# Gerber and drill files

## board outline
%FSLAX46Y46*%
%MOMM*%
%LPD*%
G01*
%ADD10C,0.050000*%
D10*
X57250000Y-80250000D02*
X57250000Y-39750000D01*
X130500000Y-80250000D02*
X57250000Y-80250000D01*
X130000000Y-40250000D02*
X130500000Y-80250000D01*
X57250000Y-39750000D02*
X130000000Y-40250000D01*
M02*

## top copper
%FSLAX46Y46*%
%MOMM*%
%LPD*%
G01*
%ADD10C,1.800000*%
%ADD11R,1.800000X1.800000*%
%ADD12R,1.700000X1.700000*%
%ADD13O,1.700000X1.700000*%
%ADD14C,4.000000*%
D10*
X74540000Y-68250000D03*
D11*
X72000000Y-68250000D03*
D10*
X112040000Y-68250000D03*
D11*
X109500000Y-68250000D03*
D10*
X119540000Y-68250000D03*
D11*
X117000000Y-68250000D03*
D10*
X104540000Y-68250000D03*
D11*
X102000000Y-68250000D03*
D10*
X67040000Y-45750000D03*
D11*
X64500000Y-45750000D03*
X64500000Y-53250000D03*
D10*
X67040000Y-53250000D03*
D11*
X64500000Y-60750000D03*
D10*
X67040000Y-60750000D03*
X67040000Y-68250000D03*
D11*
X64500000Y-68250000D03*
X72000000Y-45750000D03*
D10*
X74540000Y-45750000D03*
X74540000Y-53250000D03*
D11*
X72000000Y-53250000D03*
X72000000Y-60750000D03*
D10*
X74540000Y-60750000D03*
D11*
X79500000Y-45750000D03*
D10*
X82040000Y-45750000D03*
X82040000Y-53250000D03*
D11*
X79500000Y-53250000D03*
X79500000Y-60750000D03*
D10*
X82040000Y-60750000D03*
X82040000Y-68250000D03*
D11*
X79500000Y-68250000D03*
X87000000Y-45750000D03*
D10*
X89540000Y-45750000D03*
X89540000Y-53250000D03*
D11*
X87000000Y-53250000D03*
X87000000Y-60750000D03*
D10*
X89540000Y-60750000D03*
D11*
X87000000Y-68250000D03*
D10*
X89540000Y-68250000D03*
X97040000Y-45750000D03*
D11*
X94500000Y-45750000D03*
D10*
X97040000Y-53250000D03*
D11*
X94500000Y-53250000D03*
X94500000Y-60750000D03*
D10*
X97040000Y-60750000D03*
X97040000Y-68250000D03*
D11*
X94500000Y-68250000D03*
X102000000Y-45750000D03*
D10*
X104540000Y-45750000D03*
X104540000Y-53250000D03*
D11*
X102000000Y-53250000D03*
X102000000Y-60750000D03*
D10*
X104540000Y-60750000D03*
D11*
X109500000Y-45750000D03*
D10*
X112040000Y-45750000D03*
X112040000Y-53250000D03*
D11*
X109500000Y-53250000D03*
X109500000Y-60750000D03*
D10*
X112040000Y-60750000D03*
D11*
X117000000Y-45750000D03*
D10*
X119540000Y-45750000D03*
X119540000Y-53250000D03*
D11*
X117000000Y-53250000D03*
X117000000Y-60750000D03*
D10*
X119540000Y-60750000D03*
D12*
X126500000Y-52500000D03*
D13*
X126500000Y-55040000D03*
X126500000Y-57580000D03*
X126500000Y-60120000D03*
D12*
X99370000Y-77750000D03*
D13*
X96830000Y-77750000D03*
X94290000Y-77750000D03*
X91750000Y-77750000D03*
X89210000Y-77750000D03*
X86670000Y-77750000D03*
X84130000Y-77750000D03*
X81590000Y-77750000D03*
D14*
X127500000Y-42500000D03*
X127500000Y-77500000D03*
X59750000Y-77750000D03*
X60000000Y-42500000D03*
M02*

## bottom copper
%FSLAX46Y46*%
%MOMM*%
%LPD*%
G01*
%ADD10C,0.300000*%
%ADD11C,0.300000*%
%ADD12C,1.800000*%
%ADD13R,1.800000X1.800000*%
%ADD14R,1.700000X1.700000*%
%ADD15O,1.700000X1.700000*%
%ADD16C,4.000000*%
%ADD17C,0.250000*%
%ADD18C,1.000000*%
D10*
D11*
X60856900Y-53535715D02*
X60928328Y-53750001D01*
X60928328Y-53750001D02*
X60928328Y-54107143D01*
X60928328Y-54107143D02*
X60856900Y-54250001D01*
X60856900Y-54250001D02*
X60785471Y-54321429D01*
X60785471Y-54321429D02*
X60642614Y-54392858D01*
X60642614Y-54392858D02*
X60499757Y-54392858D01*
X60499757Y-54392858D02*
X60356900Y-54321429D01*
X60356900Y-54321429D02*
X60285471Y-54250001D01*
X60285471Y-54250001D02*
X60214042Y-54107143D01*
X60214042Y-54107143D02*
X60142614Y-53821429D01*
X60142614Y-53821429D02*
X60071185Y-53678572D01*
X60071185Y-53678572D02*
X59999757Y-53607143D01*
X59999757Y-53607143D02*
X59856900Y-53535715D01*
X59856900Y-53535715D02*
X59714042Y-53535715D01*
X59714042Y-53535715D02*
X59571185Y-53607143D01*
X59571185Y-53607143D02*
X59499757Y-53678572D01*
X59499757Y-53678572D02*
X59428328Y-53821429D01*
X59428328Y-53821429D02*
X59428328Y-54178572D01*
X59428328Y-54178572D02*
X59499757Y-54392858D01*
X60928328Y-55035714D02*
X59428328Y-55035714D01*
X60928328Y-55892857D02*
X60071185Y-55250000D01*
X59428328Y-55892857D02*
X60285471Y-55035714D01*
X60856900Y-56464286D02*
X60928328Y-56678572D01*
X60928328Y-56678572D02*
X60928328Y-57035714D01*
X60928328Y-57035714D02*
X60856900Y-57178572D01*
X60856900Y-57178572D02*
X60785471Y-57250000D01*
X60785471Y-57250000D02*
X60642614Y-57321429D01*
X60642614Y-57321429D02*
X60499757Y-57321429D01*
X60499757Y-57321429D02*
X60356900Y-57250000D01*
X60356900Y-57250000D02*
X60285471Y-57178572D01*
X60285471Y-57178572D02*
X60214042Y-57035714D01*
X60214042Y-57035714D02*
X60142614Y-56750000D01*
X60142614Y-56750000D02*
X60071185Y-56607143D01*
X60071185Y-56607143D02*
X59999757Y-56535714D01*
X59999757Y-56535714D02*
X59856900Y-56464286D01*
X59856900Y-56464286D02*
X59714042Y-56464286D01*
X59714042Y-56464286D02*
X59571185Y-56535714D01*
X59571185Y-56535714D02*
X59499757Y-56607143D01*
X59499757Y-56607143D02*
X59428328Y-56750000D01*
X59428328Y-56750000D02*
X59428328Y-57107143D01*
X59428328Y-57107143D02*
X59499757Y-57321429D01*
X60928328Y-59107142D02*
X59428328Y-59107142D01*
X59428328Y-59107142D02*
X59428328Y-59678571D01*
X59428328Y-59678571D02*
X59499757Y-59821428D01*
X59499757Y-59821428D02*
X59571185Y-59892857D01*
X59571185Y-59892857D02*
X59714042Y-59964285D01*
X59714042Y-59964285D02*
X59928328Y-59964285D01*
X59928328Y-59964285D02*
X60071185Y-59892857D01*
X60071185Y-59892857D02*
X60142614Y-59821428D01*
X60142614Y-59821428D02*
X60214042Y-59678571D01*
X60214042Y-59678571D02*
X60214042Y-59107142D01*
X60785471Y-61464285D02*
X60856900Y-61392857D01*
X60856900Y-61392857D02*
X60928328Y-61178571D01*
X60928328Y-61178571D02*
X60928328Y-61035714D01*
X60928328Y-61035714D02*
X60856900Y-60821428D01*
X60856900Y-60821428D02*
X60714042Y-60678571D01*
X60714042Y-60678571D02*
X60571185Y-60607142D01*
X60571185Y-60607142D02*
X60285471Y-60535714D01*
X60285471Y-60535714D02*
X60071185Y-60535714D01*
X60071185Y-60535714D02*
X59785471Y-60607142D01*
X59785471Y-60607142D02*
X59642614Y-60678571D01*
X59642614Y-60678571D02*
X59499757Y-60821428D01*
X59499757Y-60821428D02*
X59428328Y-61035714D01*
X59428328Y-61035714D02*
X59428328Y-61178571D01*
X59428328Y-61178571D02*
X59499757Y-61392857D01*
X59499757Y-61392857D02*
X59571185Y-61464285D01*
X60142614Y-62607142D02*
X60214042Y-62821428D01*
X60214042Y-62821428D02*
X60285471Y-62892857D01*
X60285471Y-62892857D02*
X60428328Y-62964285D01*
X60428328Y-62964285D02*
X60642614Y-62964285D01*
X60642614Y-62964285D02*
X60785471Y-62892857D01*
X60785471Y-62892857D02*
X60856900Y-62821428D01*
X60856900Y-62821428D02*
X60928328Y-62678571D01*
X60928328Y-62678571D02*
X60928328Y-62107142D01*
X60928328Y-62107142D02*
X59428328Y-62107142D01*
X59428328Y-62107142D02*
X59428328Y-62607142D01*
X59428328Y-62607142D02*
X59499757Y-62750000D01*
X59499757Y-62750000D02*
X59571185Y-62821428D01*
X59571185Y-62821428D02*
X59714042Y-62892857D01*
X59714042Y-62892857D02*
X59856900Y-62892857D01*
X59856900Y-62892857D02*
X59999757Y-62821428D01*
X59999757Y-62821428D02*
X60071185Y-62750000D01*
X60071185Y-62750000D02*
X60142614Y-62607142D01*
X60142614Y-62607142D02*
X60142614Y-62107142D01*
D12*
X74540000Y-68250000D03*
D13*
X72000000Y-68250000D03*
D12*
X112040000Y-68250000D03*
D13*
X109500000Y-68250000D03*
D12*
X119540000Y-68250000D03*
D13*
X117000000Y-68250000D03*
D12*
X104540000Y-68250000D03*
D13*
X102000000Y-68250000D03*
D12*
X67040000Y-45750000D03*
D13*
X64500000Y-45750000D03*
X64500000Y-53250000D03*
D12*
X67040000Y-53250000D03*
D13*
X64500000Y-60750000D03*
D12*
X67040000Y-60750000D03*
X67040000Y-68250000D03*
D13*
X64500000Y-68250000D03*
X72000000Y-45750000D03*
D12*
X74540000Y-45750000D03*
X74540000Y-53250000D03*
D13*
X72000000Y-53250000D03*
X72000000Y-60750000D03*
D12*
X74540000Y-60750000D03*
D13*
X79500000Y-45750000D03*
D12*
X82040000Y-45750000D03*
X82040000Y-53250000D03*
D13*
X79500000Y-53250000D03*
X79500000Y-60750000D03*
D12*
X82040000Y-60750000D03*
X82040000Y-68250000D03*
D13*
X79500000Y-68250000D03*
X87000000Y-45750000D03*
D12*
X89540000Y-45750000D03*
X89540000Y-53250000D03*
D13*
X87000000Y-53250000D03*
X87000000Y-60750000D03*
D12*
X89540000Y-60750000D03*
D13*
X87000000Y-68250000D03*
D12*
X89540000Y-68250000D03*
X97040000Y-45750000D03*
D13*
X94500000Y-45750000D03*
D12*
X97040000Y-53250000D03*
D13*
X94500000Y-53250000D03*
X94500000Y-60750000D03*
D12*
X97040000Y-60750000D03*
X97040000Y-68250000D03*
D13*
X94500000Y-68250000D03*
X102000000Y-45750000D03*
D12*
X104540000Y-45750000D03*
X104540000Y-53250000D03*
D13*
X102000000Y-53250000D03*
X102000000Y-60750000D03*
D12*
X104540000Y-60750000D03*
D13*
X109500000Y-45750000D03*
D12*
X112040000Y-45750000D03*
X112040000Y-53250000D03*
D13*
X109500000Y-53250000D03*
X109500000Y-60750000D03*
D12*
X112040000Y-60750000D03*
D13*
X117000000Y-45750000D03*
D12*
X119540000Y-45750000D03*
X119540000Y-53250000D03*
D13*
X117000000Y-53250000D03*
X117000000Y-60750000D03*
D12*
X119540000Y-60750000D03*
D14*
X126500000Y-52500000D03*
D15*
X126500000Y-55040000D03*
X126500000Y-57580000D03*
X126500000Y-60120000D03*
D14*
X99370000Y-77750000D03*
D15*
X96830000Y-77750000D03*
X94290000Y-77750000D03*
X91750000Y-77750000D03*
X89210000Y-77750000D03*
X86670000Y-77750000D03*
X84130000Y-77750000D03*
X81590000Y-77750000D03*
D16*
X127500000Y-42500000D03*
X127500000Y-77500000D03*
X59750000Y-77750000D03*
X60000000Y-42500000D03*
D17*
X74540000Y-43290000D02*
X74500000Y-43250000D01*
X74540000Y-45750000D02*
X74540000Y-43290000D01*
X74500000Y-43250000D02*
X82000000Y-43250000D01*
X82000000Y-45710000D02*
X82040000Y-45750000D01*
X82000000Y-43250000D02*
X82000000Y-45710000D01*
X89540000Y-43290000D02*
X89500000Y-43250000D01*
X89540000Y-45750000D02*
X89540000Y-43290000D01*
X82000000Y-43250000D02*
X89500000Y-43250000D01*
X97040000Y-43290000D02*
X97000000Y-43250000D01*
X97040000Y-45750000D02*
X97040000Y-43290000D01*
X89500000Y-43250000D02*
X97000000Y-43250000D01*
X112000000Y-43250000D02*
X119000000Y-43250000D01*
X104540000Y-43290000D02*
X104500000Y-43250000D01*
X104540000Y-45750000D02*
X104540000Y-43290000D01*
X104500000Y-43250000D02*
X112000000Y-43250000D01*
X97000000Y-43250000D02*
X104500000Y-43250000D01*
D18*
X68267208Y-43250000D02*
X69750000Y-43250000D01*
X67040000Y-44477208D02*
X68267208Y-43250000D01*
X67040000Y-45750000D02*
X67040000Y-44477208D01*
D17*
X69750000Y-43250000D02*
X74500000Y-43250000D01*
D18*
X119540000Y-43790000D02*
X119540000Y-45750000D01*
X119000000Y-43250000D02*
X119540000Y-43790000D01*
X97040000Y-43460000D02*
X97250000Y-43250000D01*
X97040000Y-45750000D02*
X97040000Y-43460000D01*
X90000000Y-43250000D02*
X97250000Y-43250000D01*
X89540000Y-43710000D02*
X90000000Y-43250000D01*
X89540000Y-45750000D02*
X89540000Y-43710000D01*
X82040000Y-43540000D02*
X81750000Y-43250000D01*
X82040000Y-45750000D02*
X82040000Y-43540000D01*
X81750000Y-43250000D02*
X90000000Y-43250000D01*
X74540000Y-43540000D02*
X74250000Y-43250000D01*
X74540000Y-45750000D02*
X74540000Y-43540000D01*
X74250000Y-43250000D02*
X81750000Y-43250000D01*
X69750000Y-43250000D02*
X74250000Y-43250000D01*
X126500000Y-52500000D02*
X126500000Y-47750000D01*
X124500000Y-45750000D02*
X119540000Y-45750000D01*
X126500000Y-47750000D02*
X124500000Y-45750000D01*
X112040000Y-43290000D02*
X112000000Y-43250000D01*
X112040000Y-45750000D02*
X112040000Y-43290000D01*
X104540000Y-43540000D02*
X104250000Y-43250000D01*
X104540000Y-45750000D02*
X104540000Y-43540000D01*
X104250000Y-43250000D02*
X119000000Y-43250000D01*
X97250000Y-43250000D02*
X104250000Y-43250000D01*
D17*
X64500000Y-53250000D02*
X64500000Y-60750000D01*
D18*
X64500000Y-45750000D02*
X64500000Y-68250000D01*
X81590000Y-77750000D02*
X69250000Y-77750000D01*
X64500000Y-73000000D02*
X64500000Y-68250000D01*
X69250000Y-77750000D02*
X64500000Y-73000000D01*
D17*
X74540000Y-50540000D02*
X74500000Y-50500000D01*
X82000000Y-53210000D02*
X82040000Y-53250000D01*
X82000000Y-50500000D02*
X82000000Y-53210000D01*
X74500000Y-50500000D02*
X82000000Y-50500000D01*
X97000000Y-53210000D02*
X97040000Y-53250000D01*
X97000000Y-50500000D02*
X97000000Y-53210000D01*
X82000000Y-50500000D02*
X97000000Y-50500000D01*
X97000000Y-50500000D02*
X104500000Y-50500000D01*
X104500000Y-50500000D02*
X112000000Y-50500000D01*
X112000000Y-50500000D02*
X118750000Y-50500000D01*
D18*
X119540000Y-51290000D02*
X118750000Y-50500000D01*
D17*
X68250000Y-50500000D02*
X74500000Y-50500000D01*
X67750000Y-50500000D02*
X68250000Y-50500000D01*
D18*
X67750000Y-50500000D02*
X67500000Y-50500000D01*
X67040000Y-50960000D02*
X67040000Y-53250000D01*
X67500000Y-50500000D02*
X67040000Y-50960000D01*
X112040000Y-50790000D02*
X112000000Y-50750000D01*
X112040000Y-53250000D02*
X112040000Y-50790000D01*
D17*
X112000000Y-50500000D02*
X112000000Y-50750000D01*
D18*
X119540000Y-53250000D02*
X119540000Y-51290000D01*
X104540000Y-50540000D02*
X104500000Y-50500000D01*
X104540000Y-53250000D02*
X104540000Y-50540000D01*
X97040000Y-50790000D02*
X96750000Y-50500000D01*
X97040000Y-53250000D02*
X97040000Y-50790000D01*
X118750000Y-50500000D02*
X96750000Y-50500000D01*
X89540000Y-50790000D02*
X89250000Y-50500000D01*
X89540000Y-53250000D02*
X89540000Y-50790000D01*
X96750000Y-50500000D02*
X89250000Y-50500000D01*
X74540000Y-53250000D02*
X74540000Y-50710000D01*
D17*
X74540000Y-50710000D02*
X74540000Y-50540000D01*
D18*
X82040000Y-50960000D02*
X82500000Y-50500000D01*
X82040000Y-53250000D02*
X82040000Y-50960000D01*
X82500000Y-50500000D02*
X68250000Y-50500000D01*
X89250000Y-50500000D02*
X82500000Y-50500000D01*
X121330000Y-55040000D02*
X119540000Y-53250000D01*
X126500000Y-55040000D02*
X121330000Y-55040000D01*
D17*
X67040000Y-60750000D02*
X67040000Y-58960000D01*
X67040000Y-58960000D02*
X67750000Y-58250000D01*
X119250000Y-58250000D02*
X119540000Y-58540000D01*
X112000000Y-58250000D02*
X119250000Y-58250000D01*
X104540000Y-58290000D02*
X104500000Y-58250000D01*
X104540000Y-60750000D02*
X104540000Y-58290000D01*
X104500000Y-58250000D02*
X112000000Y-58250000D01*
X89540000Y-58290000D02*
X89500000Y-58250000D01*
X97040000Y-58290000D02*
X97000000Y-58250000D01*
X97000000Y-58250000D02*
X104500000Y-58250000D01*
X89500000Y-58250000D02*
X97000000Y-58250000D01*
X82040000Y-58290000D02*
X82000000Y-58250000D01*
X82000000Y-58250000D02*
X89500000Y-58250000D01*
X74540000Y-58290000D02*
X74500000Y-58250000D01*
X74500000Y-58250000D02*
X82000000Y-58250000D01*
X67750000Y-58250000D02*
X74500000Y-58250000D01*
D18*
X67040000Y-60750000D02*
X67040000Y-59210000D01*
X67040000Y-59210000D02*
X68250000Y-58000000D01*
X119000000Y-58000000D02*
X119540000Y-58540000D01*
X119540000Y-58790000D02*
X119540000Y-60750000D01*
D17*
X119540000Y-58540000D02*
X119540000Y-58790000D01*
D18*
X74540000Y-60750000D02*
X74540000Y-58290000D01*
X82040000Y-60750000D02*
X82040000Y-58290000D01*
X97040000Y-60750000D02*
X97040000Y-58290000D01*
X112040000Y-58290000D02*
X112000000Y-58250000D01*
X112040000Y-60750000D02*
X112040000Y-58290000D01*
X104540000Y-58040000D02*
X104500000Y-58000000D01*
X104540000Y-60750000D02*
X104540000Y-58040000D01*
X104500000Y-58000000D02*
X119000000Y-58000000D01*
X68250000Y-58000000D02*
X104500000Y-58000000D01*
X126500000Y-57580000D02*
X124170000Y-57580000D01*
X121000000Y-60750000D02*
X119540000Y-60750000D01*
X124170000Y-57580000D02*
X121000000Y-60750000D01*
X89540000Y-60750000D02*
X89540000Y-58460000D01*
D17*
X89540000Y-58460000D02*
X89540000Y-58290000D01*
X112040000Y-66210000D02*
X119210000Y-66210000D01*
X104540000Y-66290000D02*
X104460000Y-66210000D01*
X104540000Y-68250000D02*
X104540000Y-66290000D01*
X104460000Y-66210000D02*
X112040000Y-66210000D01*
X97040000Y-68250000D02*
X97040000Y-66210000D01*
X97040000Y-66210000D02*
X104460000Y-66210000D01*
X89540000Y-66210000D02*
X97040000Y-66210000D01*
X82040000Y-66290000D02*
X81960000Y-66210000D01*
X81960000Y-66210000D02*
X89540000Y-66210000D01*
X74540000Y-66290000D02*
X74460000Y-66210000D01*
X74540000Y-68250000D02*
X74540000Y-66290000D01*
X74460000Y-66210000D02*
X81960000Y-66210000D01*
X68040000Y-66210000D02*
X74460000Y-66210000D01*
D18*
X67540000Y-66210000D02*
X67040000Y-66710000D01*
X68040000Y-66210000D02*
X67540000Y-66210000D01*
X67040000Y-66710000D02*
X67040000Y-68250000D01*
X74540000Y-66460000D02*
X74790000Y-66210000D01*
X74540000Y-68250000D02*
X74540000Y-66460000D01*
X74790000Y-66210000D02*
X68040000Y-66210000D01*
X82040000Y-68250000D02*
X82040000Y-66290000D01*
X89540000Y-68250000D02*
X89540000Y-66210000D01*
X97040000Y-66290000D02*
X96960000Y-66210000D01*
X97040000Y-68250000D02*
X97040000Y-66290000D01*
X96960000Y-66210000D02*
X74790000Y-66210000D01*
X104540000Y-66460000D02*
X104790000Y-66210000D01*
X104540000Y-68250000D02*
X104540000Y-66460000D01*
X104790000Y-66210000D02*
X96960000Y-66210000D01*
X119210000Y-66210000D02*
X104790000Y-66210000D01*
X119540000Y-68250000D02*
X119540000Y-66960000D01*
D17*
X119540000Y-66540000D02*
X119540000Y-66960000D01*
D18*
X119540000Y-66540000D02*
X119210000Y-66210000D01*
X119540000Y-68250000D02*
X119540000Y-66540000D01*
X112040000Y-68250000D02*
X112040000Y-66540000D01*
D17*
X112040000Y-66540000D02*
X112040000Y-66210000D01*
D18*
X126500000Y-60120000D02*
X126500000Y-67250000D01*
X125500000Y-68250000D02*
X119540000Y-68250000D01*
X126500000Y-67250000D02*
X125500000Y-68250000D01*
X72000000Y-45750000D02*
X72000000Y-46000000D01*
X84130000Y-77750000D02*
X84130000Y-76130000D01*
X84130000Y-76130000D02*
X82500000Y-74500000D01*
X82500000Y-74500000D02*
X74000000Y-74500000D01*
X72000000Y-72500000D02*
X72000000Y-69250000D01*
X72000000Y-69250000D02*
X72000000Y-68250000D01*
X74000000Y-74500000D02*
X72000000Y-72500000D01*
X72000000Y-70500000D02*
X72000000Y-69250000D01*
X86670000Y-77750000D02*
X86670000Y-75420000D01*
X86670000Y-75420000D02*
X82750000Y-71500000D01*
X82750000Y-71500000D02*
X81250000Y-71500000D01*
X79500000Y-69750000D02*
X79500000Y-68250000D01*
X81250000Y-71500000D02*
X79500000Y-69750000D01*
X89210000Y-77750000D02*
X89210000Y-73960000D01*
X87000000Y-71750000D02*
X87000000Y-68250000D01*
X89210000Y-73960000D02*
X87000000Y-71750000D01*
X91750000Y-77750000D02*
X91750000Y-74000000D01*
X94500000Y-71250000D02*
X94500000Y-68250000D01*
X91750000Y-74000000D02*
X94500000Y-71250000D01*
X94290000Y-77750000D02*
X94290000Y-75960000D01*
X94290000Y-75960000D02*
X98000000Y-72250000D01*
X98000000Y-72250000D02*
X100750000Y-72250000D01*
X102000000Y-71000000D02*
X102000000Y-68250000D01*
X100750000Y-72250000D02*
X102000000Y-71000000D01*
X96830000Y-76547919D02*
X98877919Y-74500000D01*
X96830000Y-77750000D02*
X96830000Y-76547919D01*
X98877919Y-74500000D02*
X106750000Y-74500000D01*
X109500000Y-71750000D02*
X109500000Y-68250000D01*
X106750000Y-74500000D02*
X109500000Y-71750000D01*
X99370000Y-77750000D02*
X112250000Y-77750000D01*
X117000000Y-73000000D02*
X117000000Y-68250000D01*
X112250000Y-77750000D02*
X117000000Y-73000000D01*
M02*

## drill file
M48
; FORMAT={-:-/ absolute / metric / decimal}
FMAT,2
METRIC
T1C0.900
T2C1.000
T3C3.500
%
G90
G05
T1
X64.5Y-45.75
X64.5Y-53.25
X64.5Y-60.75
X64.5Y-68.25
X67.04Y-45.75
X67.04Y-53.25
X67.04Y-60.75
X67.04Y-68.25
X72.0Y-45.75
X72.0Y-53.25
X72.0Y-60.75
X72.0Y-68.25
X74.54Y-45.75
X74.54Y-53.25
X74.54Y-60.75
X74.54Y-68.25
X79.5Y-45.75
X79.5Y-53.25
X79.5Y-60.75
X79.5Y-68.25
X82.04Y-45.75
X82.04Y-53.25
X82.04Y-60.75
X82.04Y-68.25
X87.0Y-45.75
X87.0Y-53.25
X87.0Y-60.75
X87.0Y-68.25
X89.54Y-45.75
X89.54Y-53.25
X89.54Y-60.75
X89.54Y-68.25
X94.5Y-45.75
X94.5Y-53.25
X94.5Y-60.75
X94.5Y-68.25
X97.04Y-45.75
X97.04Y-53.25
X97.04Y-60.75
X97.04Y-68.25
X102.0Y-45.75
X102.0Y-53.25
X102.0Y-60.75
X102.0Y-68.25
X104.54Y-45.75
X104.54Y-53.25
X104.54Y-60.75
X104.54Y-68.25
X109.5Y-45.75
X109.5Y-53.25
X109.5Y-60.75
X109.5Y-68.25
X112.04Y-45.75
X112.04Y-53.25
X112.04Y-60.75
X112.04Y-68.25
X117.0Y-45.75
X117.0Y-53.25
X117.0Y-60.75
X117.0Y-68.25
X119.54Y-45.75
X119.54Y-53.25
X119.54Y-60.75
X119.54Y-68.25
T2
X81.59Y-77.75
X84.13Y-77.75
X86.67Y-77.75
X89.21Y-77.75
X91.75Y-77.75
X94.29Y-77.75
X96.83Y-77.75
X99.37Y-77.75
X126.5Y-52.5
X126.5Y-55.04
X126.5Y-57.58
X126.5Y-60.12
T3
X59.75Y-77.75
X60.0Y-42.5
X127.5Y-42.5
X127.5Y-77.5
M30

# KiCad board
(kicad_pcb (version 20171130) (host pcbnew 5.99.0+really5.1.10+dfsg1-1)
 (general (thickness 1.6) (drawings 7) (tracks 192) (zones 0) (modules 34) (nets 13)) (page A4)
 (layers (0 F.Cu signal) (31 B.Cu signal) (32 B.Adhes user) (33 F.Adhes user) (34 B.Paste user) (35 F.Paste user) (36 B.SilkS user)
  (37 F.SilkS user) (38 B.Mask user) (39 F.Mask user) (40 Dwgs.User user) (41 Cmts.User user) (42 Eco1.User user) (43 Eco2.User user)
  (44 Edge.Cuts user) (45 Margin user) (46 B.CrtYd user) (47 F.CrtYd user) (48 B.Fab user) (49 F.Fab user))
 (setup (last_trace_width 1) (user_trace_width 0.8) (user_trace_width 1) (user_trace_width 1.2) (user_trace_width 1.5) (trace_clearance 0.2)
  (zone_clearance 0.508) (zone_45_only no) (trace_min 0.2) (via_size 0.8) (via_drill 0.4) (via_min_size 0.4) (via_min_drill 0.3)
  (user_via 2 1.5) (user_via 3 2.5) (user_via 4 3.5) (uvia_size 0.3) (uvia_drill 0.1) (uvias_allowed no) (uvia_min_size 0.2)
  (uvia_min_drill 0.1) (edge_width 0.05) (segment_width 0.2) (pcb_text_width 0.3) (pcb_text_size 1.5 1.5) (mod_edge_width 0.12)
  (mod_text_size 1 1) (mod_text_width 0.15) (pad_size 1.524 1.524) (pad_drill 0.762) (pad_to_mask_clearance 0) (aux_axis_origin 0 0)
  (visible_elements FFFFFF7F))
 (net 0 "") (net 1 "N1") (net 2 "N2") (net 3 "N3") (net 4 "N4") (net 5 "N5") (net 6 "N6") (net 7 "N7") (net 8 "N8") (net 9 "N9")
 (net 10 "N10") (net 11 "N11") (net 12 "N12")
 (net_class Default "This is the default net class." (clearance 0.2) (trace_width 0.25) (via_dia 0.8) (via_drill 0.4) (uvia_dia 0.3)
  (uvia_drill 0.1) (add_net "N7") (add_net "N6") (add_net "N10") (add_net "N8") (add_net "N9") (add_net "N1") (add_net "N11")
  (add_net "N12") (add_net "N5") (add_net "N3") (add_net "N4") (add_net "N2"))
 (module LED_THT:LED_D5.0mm (layer F.Cu) (at 72 68.25)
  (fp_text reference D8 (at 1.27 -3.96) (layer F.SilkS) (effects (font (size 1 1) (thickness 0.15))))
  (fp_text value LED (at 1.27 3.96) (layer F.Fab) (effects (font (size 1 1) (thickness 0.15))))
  (pad 2 thru_hole circle (at 2.54 0) (size 1.8 1.8) (drill 0.9) (layers *.Cu *.Mask) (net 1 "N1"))
  (pad 1 thru_hole rect (at 0 0) (size 1.8 1.8) (drill 0.9) (layers *.Cu *.Mask) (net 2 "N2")))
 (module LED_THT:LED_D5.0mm (layer F.Cu) (at 109.5 68.25)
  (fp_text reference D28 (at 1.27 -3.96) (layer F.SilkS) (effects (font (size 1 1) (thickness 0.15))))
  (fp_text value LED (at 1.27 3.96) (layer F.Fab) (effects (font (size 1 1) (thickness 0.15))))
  (pad 2 thru_hole circle (at 2.54 0) (size 1.8 1.8) (drill 0.9) (layers *.Cu *.Mask) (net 1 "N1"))
  (pad 1 thru_hole rect (at 0 0) (size 1.8 1.8) (drill 0.9) (layers *.Cu *.Mask) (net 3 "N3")))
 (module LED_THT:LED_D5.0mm (layer F.Cu) (at 117 68.25)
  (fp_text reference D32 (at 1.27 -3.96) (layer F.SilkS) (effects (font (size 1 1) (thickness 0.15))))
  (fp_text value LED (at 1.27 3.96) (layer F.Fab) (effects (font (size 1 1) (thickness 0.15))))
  (pad 2 thru_hole circle (at 2.54 0) (size 1.8 1.8) (drill 0.9) (layers *.Cu *.Mask) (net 1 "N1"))
  (pad 1 thru_hole rect (at 0 0) (size 1.8 1.8) (drill 0.9) (layers *.Cu *.Mask) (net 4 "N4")))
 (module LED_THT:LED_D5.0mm (layer F.Cu) (at 102 68.25)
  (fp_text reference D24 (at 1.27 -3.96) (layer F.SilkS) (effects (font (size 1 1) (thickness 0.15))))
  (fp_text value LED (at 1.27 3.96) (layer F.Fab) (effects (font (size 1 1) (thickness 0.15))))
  (pad 2 thru_hole circle (at 2.54 0) (size 1.8 1.8) (drill 0.9) (layers *.Cu *.Mask) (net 1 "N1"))
  (pad 1 thru_hole rect (at 0 0) (size 1.8 1.8) (drill 0.9) (layers *.Cu *.Mask) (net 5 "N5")))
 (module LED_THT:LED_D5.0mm (layer F.Cu) (at 64.5 45.75)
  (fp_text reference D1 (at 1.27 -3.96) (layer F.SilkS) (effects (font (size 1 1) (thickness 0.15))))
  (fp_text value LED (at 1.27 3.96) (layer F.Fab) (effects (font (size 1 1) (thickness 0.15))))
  (pad 2 thru_hole circle (at 2.54 0) (size 1.8 1.8) (drill 0.9) (layers *.Cu *.Mask) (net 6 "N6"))
  (pad 1 thru_hole rect (at 0 0) (size 1.8 1.8) (drill 0.9) (layers *.Cu *.Mask) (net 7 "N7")))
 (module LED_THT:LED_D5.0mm (layer F.Cu) (at 64.5 53.25)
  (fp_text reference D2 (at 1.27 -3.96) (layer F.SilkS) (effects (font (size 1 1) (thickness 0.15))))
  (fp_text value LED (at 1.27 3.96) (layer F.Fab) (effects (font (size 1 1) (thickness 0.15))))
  (pad 1 thru_hole rect (at 0 0) (size 1.8 1.8) (drill 0.9) (layers *.Cu *.Mask) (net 7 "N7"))
  (pad 2 thru_hole circle (at 2.54 0) (size 1.8 1.8) (drill 0.9) (layers *.Cu *.Mask) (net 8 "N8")))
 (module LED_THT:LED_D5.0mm (layer F.Cu) (at 64.5 60.75)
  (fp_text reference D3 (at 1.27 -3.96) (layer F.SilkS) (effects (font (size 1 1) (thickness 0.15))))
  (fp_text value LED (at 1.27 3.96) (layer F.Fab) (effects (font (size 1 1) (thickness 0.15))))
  (pad 1 thru_hole rect (at 0 0) (size 1.8 1.8) (drill 0.9) (layers *.Cu *.Mask) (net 7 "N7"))
  (pad 2 thru_hole circle (at 2.54 0) (size 1.8 1.8) (drill 0.9) (layers *.Cu *.Mask) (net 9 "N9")))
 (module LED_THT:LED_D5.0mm (layer F.Cu) (at 64.5 68.25)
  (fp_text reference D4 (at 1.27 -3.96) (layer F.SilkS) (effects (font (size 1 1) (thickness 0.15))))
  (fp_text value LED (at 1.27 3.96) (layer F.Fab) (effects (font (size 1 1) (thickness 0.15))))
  (pad 2 thru_hole circle (at 2.54 0) (size 1.8 1.8) (drill 0.9) (layers *.Cu *.Mask) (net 1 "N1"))
  (pad 1 thru_hole rect (at 0 0) (size 1.8 1.8) (drill 0.9) (layers *.Cu *.Mask) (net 7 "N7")))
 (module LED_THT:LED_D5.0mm (layer F.Cu) (at 72 45.75)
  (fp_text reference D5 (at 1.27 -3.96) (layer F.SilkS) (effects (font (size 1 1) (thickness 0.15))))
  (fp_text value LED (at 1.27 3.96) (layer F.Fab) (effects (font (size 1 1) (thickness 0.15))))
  (pad 1 thru_hole rect (at 0 0) (size 1.8 1.8) (drill 0.9) (layers *.Cu *.Mask) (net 2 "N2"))
  (pad 2 thru_hole circle (at 2.54 0) (size 1.8 1.8) (drill 0.9) (layers *.Cu *.Mask) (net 6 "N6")))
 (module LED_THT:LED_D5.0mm (layer F.Cu) (at 72 53.25)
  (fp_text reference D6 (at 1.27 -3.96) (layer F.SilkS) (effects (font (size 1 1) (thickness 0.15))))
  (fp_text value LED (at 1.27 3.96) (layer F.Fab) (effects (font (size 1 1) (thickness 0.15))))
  (pad 2 thru_hole circle (at 2.54 0) (size 1.8 1.8) (drill 0.9) (layers *.Cu *.Mask) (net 8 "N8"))
  (pad 1 thru_hole rect (at 0 0) (size 1.8 1.8) (drill 0.9) (layers *.Cu *.Mask) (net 2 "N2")))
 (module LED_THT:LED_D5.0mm (layer F.Cu) (at 72 60.75)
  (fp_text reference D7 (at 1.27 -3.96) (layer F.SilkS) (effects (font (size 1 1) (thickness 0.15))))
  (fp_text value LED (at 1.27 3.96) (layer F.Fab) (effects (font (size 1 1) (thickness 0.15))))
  (pad 1 thru_hole rect (at 0 0) (size 1.8 1.8) (drill 0.9) (layers *.Cu *.Mask) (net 2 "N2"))
  (pad 2 thru_hole circle (at 2.54 0) (size 1.8 1.8) (drill 0.9) (layers *.Cu *.Mask) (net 9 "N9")))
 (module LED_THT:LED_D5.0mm (layer F.Cu) (at 79.5 45.75)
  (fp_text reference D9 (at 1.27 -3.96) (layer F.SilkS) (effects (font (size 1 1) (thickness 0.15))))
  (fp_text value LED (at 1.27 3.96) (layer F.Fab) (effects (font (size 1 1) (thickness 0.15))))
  (pad 1 thru_hole rect (at 0 0) (size 1.8 1.8) (drill 0.9) (layers *.Cu *.Mask) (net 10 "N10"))
  (pad 2 thru_hole circle (at 2.54 0) (size 1.8 1.8) (drill 0.9) (layers *.Cu *.Mask) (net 6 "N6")))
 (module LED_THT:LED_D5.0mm (layer F.Cu) (at 79.5 53.25)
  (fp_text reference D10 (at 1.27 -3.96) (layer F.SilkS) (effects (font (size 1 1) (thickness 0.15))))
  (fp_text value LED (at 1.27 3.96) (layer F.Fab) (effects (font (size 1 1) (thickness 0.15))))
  (pad 2 thru_hole circle (at 2.54 0) (size 1.8 1.8) (drill 0.9) (layers *.Cu *.Mask) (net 8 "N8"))
  (pad 1 thru_hole rect (at 0 0) (size 1.8 1.8) (drill 0.9) (layers *.Cu *.Mask) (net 10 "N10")))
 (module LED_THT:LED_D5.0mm (layer F.Cu) (at 79.5 60.75)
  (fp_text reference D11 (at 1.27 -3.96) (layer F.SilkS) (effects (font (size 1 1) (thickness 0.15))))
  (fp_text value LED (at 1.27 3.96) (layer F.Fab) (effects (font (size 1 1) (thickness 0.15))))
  (pad 1 thru_hole rect (at 0 0) (size 1.8 1.8) (drill 0.9) (layers *.Cu *.Mask) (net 10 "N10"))
  (pad 2 thru_hole circle (at 2.54 0) (size 1.8 1.8) (drill 0.9) (layers *.Cu *.Mask) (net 9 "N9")))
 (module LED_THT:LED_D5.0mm (layer F.Cu) (at 79.5 68.25)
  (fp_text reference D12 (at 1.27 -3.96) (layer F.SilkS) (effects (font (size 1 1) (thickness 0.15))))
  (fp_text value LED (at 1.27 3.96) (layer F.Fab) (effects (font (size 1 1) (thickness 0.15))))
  (pad 2 thru_hole circle (at 2.54 0) (size 1.8 1.8) (drill 0.9) (layers *.Cu *.Mask) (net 1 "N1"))
  (pad 1 thru_hole rect (at 0 0) (size 1.8 1.8) (drill 0.9) (layers *.Cu *.Mask) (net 10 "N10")))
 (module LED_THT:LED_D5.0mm (layer F.Cu) (at 87 45.75)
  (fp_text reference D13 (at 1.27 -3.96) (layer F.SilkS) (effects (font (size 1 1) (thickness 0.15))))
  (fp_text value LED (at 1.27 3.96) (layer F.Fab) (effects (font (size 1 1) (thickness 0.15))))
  (pad 1 thru_hole rect (at 0 0) (size 1.8 1.8) (drill 0.9) (layers *.Cu *.Mask) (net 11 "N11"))
  (pad 2 thru_hole circle (at 2.54 0) (size 1.8 1.8) (drill 0.9) (layers *.Cu *.Mask) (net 6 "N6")))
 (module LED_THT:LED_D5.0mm (layer F.Cu) (at 87 53.25)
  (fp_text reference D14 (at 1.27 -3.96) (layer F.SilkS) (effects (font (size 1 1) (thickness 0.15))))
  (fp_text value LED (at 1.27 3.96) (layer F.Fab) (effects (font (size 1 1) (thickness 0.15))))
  (pad 2 thru_hole circle (at 2.54 0) (size 1.8 1.8) (drill 0.9) (layers *.Cu *.Mask) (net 8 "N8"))
  (pad 1 thru_hole rect (at 0 0) (size 1.8 1.8) (drill 0.9) (layers *.Cu *.Mask) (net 11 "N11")))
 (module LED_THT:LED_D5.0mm (layer F.Cu) (at 87 60.75)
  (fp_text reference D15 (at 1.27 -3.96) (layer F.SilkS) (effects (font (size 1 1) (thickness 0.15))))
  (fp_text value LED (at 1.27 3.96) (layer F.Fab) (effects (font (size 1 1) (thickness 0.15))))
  (pad 1 thru_hole rect (at 0 0) (size 1.8 1.8) (drill 0.9) (layers *.Cu *.Mask) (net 11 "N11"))
  (pad 2 thru_hole circle (at 2.54 0) (size 1.8 1.8) (drill 0.9) (layers *.Cu *.Mask) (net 9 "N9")))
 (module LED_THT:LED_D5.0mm (layer F.Cu) (at 87 68.25)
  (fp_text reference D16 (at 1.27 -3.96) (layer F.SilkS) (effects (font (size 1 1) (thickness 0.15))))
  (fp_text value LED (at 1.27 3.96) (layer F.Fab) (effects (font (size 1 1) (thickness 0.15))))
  (pad 1 thru_hole rect (at 0 0) (size 1.8 1.8) (drill 0.9) (layers *.Cu *.Mask) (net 11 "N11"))
  (pad 2 thru_hole circle (at 2.54 0) (size 1.8 1.8) (drill 0.9) (layers *.Cu *.Mask) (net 1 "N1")))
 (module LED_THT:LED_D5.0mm (layer F.Cu) (at 94.5 45.75)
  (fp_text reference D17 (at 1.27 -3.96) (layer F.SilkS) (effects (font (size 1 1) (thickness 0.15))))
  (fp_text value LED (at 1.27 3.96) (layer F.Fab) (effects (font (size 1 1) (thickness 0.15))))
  (pad 2 thru_hole circle (at 2.54 0) (size 1.8 1.8) (drill 0.9) (layers *.Cu *.Mask) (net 6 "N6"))
  (pad 1 thru_hole rect (at 0 0) (size 1.8 1.8) (drill 0.9) (layers *.Cu *.Mask) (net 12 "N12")))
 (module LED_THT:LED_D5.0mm (layer F.Cu) (at 94.5 53.25)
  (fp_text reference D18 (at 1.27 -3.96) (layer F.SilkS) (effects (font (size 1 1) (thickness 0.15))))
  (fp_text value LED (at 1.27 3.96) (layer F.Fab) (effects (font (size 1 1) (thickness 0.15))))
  (pad 2 thru_hole circle (at 2.54 0) (size 1.8 1.8) (drill 0.9) (layers *.Cu *.Mask) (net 8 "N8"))
  (pad 1 thru_hole rect (at 0 0) (size 1.8 1.8) (drill 0.9) (layers *.Cu *.Mask) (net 12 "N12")))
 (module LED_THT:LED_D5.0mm (layer F.Cu) (at 94.5 60.75)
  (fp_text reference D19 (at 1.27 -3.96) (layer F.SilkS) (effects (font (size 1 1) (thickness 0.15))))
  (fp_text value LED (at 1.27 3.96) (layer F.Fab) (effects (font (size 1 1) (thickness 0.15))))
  (pad 1 thru_hole rect (at 0 0) (size 1.8 1.8) (drill 0.9) (layers *.Cu *.Mask) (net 12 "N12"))
  (pad 2 thru_hole circle (at 2.54 0) (size 1.8 1.8) (drill 0.9) (layers *.Cu *.Mask) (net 9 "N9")))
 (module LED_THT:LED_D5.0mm (layer F.Cu) (at 94.5 68.25)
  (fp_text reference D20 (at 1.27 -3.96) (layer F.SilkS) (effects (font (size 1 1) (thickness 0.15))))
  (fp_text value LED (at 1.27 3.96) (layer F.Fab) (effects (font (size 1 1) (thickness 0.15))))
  (pad 2 thru_hole circle (at 2.54 0) (size 1.8 1.8) (drill 0.9) (layers *.Cu *.Mask) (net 1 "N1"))
  (pad 1 thru_hole rect (at 0 0) (size 1.8 1.8) (drill 0.9) (layers *.Cu *.Mask) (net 12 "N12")))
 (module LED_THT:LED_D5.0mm (layer F.Cu) (at 102 45.75)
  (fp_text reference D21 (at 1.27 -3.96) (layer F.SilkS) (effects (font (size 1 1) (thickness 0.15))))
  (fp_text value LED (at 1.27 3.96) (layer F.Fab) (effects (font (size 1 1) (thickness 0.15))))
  (pad 1 thru_hole rect (at 0 0) (size 1.8 1.8) (drill 0.9) (layers *.Cu *.Mask) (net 5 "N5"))
  (pad 2 thru_hole circle (at 2.54 0) (size 1.8 1.8) (drill 0.9) (layers *.Cu *.Mask) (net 6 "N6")))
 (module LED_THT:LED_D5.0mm (layer F.Cu) (at 102 53.25)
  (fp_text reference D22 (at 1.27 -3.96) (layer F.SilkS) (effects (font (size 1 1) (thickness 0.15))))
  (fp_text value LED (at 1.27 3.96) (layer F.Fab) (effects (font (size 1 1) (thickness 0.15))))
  (pad 2 thru_hole circle (at 2.54 0) (size 1.8 1.8) (drill 0.9) (layers *.Cu *.Mask) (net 8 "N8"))
  (pad 1 thru_hole rect (at 0 0) (size 1.8 1.8) (drill 0.9) (layers *.Cu *.Mask) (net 5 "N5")))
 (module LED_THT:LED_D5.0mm (layer F.Cu) (at 102 60.75)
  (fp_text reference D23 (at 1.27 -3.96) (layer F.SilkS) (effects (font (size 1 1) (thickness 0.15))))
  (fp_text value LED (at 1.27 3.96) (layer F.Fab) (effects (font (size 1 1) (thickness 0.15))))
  (pad 1 thru_hole rect (at 0 0) (size 1.8 1.8) (drill 0.9) (layers *.Cu *.Mask) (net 5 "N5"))
  (pad 2 thru_hole circle (at 2.54 0) (size 1.8 1.8) (drill 0.9) (layers *.Cu *.Mask) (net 9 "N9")))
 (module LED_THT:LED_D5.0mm (layer F.Cu) (at 109.5 45.75)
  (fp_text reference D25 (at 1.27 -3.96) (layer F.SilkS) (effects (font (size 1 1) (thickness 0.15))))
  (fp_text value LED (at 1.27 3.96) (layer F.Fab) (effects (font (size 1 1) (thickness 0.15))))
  (pad 1 thru_hole rect (at 0 0) (size 1.8 1.8) (drill 0.9) (layers *.Cu *.Mask) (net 3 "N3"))
  (pad 2 thru_hole circle (at 2.54 0) (size 1.8 1.8) (drill 0.9) (layers *.Cu *.Mask) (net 6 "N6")))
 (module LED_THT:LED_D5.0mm (layer F.Cu) (at 109.5 53.25)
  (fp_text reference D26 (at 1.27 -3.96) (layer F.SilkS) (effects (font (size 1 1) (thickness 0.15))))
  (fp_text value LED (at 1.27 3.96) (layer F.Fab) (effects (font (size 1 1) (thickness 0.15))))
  (pad 2 thru_hole circle (at 2.54 0) (size 1.8 1.8) (drill 0.9) (layers *.Cu *.Mask) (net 8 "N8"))
  (pad 1 thru_hole rect (at 0 0) (size 1.8 1.8) (drill 0.9) (layers *.Cu *.Mask) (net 3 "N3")))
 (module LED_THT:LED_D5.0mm (layer F.Cu) (at 109.5 60.75)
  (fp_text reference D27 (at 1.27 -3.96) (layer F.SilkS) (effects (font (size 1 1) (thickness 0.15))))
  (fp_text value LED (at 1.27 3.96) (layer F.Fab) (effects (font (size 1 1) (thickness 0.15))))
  (pad 1 thru_hole rect (at 0 0) (size 1.8 1.8) (drill 0.9) (layers *.Cu *.Mask) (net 3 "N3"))
  (pad 2 thru_hole circle (at 2.54 0) (size 1.8 1.8) (drill 0.9) (layers *.Cu *.Mask) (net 9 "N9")))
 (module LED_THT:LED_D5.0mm (layer F.Cu) (at 117 45.75)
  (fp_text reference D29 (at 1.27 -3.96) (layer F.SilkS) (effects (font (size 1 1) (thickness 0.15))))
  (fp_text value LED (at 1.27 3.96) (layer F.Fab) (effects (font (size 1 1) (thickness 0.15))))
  (pad 1 thru_hole rect (at 0 0) (size 1.8 1.8) (drill 0.9) (layers *.Cu *.Mask) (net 4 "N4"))
  (pad 2 thru_hole circle (at 2.54 0) (size 1.8 1.8) (drill 0.9) (layers *.Cu *.Mask) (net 6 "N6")))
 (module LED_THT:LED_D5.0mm (layer F.Cu) (at 117 53.25)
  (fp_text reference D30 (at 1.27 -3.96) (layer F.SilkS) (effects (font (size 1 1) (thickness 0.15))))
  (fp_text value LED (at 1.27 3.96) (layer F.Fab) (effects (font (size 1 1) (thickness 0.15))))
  (pad 2 thru_hole circle (at 2.54 0) (size 1.8 1.8) (drill 0.9) (layers *.Cu *.Mask) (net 8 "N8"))
  (pad 1 thru_hole rect (at 0 0) (size 1.8 1.8) (drill 0.9) (layers *.Cu *.Mask) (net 4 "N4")))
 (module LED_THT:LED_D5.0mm (layer F.Cu) (at 117 60.75)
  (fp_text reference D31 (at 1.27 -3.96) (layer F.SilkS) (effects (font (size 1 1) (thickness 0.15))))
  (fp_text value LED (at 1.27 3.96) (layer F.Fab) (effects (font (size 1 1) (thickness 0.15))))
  (pad 1 thru_hole rect (at 0 0) (size 1.8 1.8) (drill 0.9) (layers *.Cu *.Mask) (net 4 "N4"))
  (pad 2 thru_hole circle (at 2.54 0) (size 1.8 1.8) (drill 0.9) (layers *.Cu *.Mask) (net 9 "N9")))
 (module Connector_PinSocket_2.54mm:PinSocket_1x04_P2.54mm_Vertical (layer F.Cu) (at 126.5 52.5)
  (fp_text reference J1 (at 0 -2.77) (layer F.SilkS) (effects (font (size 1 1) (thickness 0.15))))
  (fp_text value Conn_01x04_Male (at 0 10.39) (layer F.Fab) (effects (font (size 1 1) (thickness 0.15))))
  (pad 1 thru_hole rect (at 0 0) (size 1.7 1.7) (drill 1) (layers *.Cu *.Mask) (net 6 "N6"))
  (pad 2 thru_hole oval (at 0 2.54) (size 1.7 1.7) (drill 1) (layers *.Cu *.Mask) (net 8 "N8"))
  (pad 3 thru_hole oval (at 0 5.08) (size 1.7 1.7) (drill 1) (layers *.Cu *.Mask) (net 9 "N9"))
  (pad 4 thru_hole oval (at 0 7.62) (size 1.7 1.7) (drill 1) (layers *.Cu *.Mask) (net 1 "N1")))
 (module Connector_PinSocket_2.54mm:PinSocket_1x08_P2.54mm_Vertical (layer F.Cu) (at 99.37 77.75 270)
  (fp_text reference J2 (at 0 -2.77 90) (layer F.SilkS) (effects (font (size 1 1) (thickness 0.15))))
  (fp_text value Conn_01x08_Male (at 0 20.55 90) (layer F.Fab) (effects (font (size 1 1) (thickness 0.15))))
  (pad 1 thru_hole rect (at 0 0 270) (size 1.7 1.7) (drill 1) (layers *.Cu *.Mask) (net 4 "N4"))
  (pad 2 thru_hole oval (at 0 2.54 270) (size 1.7 1.7) (drill 1) (layers *.Cu *.Mask) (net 3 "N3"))
  (pad 3 thru_hole oval (at 0 5.08 270) (size 1.7 1.7) (drill 1) (layers *.Cu *.Mask) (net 5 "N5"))
  (pad 4 thru_hole oval (at 0 7.62 270) (size 1.7 1.7) (drill 1) (layers *.Cu *.Mask) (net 12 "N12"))
  (pad 5 thru_hole oval (at 0 10.16 270) (size 1.7 1.7) (drill 1) (layers *.Cu *.Mask) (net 11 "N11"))
  (pad 6 thru_hole oval (at 0 12.7 270) (size 1.7 1.7) (drill 1) (layers *.Cu *.Mask) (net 10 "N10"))
  (pad 7 thru_hole oval (at 0 15.24 270) (size 1.7 1.7) (drill 1) (layers *.Cu *.Mask) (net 2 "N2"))
  (pad 8 thru_hole oval (at 0 17.78 270) (size 1.7 1.7) (drill 1) (layers *.Cu *.Mask) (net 7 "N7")))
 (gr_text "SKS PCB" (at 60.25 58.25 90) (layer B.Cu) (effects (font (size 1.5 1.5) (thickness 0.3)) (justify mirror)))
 (gr_line (start 57.25 80.25) (end 57.25 39.75) (layer Edge.Cuts) (width 0.05))
 (gr_line (start 130.5 80.25) (end 57.25 80.25) (layer Edge.Cuts) (width 0.05))
 (gr_line (start 130 40.25) (end 130.5 80.25) (layer Edge.Cuts) (width 0.05))
 (gr_line (start 57.25 39.75) (end 130 40.25) (layer Edge.Cuts) (width 0.05))
 (via (at 127.5 42.5) (size 4) (drill 3.5) (layers F.Cu B.Cu) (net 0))
 (via (at 127.5 77.5) (size 4) (drill 3.5) (layers F.Cu B.Cu) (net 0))
 (via (at 59.75 77.75) (size 4) (drill 3.5) (layers F.Cu B.Cu) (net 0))
 (via (at 60 42.5) (size 4) (drill 3.5) (layers F.Cu B.Cu) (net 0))
 (segment (start 74.54 43.29) (end 74.5 43.25) (width 0.25) (layer B.Cu) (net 6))
 (segment (start 74.54 45.75) (end 74.54 43.29) (width 0.25) (layer B.Cu) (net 6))
 (segment (start 74.5 43.25) (end 82 43.25) (width 0.25) (layer B.Cu) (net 6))
 (segment (start 82 45.71) (end 82.04 45.75) (width 0.25) (layer B.Cu) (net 6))
 (segment (start 82 43.25) (end 82 45.71) (width 0.25) (layer B.Cu) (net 6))
 (segment (start 89.54 43.29) (end 89.5 43.25) (width 0.25) (layer B.Cu) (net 6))
 (segment (start 89.54 45.75) (end 89.54 43.29) (width 0.25) (layer B.Cu) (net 6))
 (segment (start 82 43.25) (end 89.5 43.25) (width 0.25) (layer B.Cu) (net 6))
 (segment (start 97.04 43.29) (end 97 43.25) (width 0.25) (layer B.Cu) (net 6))
 (segment (start 97.04 45.75) (end 97.04 43.29) (width 0.25) (layer B.Cu) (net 6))
 (segment (start 89.5 43.25) (end 97 43.25) (width 0.25) (layer B.Cu) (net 6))
 (segment (start 112 43.25) (end 119 43.25) (width 0.25) (layer B.Cu) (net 6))
 (segment (start 104.54 43.29) (end 104.5 43.25) (width 0.25) (layer B.Cu) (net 6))
 (segment (start 104.54 45.75) (end 104.54 43.29) (width 0.25) (layer B.Cu) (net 6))
 (segment (start 104.5 43.25) (end 112 43.25) (width 0.25) (layer B.Cu) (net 6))
 (segment (start 97 43.25) (end 104.5 43.25) (width 0.25) (layer B.Cu) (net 6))
 (segment (start 68.267208 43.25) (end 69.75 43.25) (width 1) (layer B.Cu) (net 6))
 (segment (start 67.04 44.477208) (end 68.267208 43.25) (width 1) (layer B.Cu) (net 6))
 (segment (start 67.04 45.75) (end 67.04 44.477208) (width 1) (layer B.Cu) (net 6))
 (segment (start 69.75 43.25) (end 74.5 43.25) (width 0.25) (layer B.Cu) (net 6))
 (segment (start 119.54 43.79) (end 119.54 45.75) (width 1) (layer B.Cu) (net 6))
 (segment (start 119 43.25) (end 119.54 43.79) (width 1) (layer B.Cu) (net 6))
 (segment (start 97.04 43.46) (end 97.25 43.25) (width 1) (layer B.Cu) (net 6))
 (segment (start 97.04 45.75) (end 97.04 43.46) (width 1) (layer B.Cu) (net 6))
 (segment (start 90 43.25) (end 97.25 43.25) (width 1) (layer B.Cu) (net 6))
 (segment (start 89.54 43.71) (end 90 43.25) (width 1) (layer B.Cu) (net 6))
 (segment (start 89.54 45.75) (end 89.54 43.71) (width 1) (layer B.Cu) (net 6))
 (segment (start 82.04 43.54) (end 81.75 43.25) (width 1) (layer B.Cu) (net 6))
 (segment (start 82.04 45.75) (end 82.04 43.54) (width 1) (layer B.Cu) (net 6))
 (segment (start 81.75 43.25) (end 90 43.25) (width 1) (layer B.Cu) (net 6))
 (segment (start 74.54 43.54) (end 74.25 43.25) (width 1) (layer B.Cu) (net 6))
 (segment (start 74.54 45.75) (end 74.54 43.54) (width 1) (layer B.Cu) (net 6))
 (segment (start 74.25 43.25) (end 81.75 43.25) (width 1) (layer B.Cu) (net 6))
 (segment (start 69.75 43.25) (end 74.25 43.25) (width 1) (layer B.Cu) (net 6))
 (segment (start 126.5 52.5) (end 126.5 47.75) (width 1) (layer B.Cu) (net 6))
 (segment (start 124.5 45.75) (end 119.54 45.75) (width 1) (layer B.Cu) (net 6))
 (segment (start 126.5 47.75) (end 124.5 45.75) (width 1) (layer B.Cu) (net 6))
 (segment (start 112.04 43.29) (end 112 43.25) (width 1) (layer B.Cu) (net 6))
 (segment (start 112.04 45.75) (end 112.04 43.29) (width 1) (layer B.Cu) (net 6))
 (segment (start 104.54 43.54) (end 104.25 43.25) (width 1) (layer B.Cu) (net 6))
 (segment (start 104.54 45.75) (end 104.54 43.54) (width 1) (layer B.Cu) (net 6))
 (segment (start 104.25 43.25) (end 119 43.25) (width 1) (layer B.Cu) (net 6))
 (segment (start 97.25 43.25) (end 104.25 43.25) (width 1) (layer B.Cu) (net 6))
 (segment (start 64.5 53.25) (end 64.5 60.75) (width 0.25) (layer B.Cu) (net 7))
 (segment (start 64.5 45.75) (end 64.5 68.25) (width 1) (layer B.Cu) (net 7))
 (segment (start 81.59 77.75) (end 69.25 77.75) (width 1) (layer B.Cu) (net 7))
 (segment (start 64.5 73) (end 64.5 68.25) (width 1) (layer B.Cu) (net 7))
 (segment (start 69.25 77.75) (end 64.5 73) (width 1) (layer B.Cu) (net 7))
 (segment (start 74.54 50.54) (end 74.5 50.5) (width 0.25) (layer B.Cu) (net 8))
 (segment (start 82 53.21) (end 82.04 53.25) (width 0.25) (layer B.Cu) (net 8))
 (segment (start 82 50.5) (end 82 53.21) (width 0.25) (layer B.Cu) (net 8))
 (segment (start 74.5 50.5) (end 82 50.5) (width 0.25) (layer B.Cu) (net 8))
 (segment (start 97 53.21) (end 97.04 53.25) (width 0.25) (layer B.Cu) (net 8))
 (segment (start 97 50.5) (end 97 53.21) (width 0.25) (layer B.Cu) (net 8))
 (segment (start 82 50.5) (end 97 50.5) (width 0.25) (layer B.Cu) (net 8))
 (segment (start 97 50.5) (end 104.5 50.5) (width 0.25) (layer B.Cu) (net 8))
 (segment (start 104.5 50.5) (end 112 50.5) (width 0.25) (layer B.Cu) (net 8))
 (segment (start 112 50.5) (end 118.75 50.5) (width 0.25) (layer B.Cu) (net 8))
 (segment (start 119.54 51.29) (end 118.75 50.5) (width 1) (layer B.Cu) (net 8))
 (segment (start 68.25 50.5) (end 74.5 50.5) (width 0.25) (layer B.Cu) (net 8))
 (segment (start 67.75 50.5) (end 68.25 50.5) (width 0.25) (layer B.Cu) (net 8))
 (segment (start 67.75 50.5) (end 67.5 50.5) (width 1) (layer B.Cu) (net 8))
 (segment (start 67.04 50.96) (end 67.04 53.25) (width 1) (layer B.Cu) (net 8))
 (segment (start 67.5 50.5) (end 67.04 50.96) (width 1) (layer B.Cu) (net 8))
 (segment (start 112.04 50.79) (end 112 50.75) (width 1) (layer B.Cu) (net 8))
 (segment (start 112.04 53.25) (end 112.04 50.79) (width 1) (layer B.Cu) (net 8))
 (segment (start 112 50.5) (end 112 50.75) (width 0.25) (layer B.Cu) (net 8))
 (segment (start 119.54 53.25) (end 119.54 51.29) (width 1) (layer B.Cu) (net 8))
 (segment (start 104.54 50.54) (end 104.5 50.5) (width 1) (layer B.Cu) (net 8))
 (segment (start 104.54 53.25) (end 104.54 50.54) (width 1) (layer B.Cu) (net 8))
 (segment (start 97.04 50.79) (end 96.75 50.5) (width 1) (layer B.Cu) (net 8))
 (segment (start 97.04 53.25) (end 97.04 50.79) (width 1) (layer B.Cu) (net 8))
 (segment (start 118.75 50.5) (end 96.75 50.5) (width 1) (layer B.Cu) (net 8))
 (segment (start 89.54 50.79) (end 89.25 50.5) (width 1) (layer B.Cu) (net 8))
 (segment (start 89.54 53.25) (end 89.54 50.79) (width 1) (layer B.Cu) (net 8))
 (segment (start 96.75 50.5) (end 89.25 50.5) (width 1) (layer B.Cu) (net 8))
 (segment (start 74.54 53.25) (end 74.54 50.71) (width 1) (layer B.Cu) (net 8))
 (segment (start 74.54 50.71) (end 74.54 50.54) (width 0.25) (layer B.Cu) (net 8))
 (segment (start 82.04 50.96) (end 82.5 50.5) (width 1) (layer B.Cu) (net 8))
 (segment (start 82.04 53.25) (end 82.04 50.96) (width 1) (layer B.Cu) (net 8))
 (segment (start 82.5 50.5) (end 68.25 50.5) (width 1) (layer B.Cu) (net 8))
 (segment (start 89.25 50.5) (end 82.5 50.5) (width 1) (layer B.Cu) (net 8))
 (segment (start 121.33 55.04) (end 119.54 53.25) (width 1) (layer B.Cu) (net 8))
 (segment (start 126.5 55.04) (end 121.33 55.04) (width 1) (layer B.Cu) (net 8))
 (segment (start 67.04 60.75) (end 67.04 58.96) (width 0.25) (layer B.Cu) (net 9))
 (segment (start 67.04 58.96) (end 67.75 58.25) (width 0.25) (layer B.Cu) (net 9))
 (segment (start 119.25 58.25) (end 119.54 58.54) (width 0.25) (layer B.Cu) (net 9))
 (segment (start 112 58.25) (end 119.25 58.25) (width 0.25) (layer B.Cu) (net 9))
 (segment (start 104.54 58.29) (end 104.5 58.25) (width 0.25) (layer B.Cu) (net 9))
 (segment (start 104.54 60.75) (end 104.54 58.29) (width 0.25) (layer B.Cu) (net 9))
 (segment (start 104.5 58.25) (end 112 58.25) (width 0.25) (layer B.Cu) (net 9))
 (segment (start 89.54 58.29) (end 89.5 58.25) (width 0.25) (layer B.Cu) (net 9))
 (segment (start 97.04 58.29) (end 97 58.25) (width 0.25) (layer B.Cu) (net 9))
 (segment (start 97 58.25) (end 104.5 58.25) (width 0.25) (layer B.Cu) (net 9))
 (segment (start 89.5 58.25) (end 97 58.25) (width 0.25) (layer B.Cu) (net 9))
 (segment (start 82.04 58.29) (end 82 58.25) (width 0.25) (layer B.Cu) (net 9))
 (segment (start 82 58.25) (end 89.5 58.25) (width 0.25) (layer B.Cu) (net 9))
 (segment (start 74.54 58.29) (end 74.5 58.25) (width 0.25) (layer B.Cu) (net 9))
 (segment (start 74.5 58.25) (end 82 58.25) (width 0.25) (layer B.Cu) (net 9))
 (segment (start 67.75 58.25) (end 74.5 58.25) (width 0.25) (layer B.Cu) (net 9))
 (segment (start 67.04 60.75) (end 67.04 59.21) (width 1) (layer B.Cu) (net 9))
 (segment (start 67.04 59.21) (end 68.25 58) (width 1) (layer B.Cu) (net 9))
 (segment (start 119 58) (end 119.54 58.54) (width 1) (layer B.Cu) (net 9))
 (segment (start 119.54 58.79) (end 119.54 60.75) (width 1) (layer B.Cu) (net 9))
 (segment (start 119.54 58.54) (end 119.54 58.79) (width 0.25) (layer B.Cu) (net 9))
 (segment (start 74.54 60.75) (end 74.54 58.29) (width 1) (layer B.Cu) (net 9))
 (segment (start 82.04 60.75) (end 82.04 58.29) (width 1) (layer B.Cu) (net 9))
 (segment (start 97.04 60.75) (end 97.04 58.29) (width 1) (layer B.Cu) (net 9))
 (segment (start 112.04 58.29) (end 112 58.25) (width 1) (layer B.Cu) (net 9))
 (segment (start 112.04 60.75) (end 112.04 58.29) (width 1) (layer B.Cu) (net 9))
 (segment (start 104.54 58.04) (end 104.5 58) (width 1) (layer B.Cu) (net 9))
 (segment (start 104.54 60.75) (end 104.54 58.04) (width 1) (layer B.Cu) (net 9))
 (segment (start 104.5 58) (end 119 58) (width 1) (layer B.Cu) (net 9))
 (segment (start 68.25 58) (end 104.5 58) (width 1) (layer B.Cu) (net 9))
 (segment (start 126.5 57.58) (end 124.17 57.58) (width 1) (layer B.Cu) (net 9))
 (segment (start 121 60.75) (end 119.54 60.75) (width 1) (layer B.Cu) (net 9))
 (segment (start 124.17 57.58) (end 121 60.75) (width 1) (layer B.Cu) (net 9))
 (segment (start 89.54 60.75) (end 89.54 58.46) (width 1) (layer B.Cu) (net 9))
 (segment (start 89.54 58.46) (end 89.54 58.29) (width 0.25) (layer B.Cu) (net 9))
 (segment (start 112.04 66.21) (end 119.21 66.21) (width 0.25) (layer B.Cu) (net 1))
 (segment (start 104.54 66.29) (end 104.46 66.21) (width 0.25) (layer B.Cu) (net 1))
 (segment (start 104.54 68.25) (end 104.54 66.29) (width 0.25) (layer B.Cu) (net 1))
 (segment (start 104.46 66.21) (end 112.04 66.21) (width 0.25) (layer B.Cu) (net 1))
 (segment (start 97.04 68.25) (end 97.04 66.21) (width 0.25) (layer B.Cu) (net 1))
 (segment (start 97.04 66.21) (end 104.46 66.21) (width 0.25) (layer B.Cu) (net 1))
 (segment (start 89.54 66.21) (end 97.04 66.21) (width 0.25) (layer B.Cu) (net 1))
 (segment (start 82.04 66.29) (end 81.96 66.21) (width 0.25) (layer B.Cu) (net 1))
 (segment (start 81.96 66.21) (end 89.54 66.21) (width 0.25) (layer B.Cu) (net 1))
 (segment (start 74.54 66.29) (end 74.46 66.21) (width 0.25) (layer B.Cu) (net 1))
 (segment (start 74.54 68.25) (end 74.54 66.29) (width 0.25) (layer B.Cu) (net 1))
 (segment (start 74.46 66.21) (end 81.96 66.21) (width 0.25) (layer B.Cu) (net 1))
 (segment (start 68.04 66.21) (end 74.46 66.21) (width 0.25) (layer B.Cu) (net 1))
 (segment (start 67.54 66.21) (end 67.04 66.71) (width 1) (layer B.Cu) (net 1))
 (segment (start 68.04 66.21) (end 67.54 66.21) (width 1) (layer B.Cu) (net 1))
 (segment (start 67.04 66.71) (end 67.04 68.25) (width 1) (layer B.Cu) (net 1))
 (segment (start 74.54 66.46) (end 74.79 66.21) (width 1) (layer B.Cu) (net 1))
 (segment (start 74.54 68.25) (end 74.54 66.46) (width 1) (layer B.Cu) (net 1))
 (segment (start 74.79 66.21) (end 68.04 66.21) (width 1) (layer B.Cu) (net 1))
 (segment (start 82.04 68.25) (end 82.04 66.29) (width 1) (layer B.Cu) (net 1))
 (segment (start 89.54 68.25) (end 89.54 66.21) (width 1) (layer B.Cu) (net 1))
 (segment (start 97.04 66.29) (end 96.96 66.21) (width 1) (layer B.Cu) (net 1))
 (segment (start 97.04 68.25) (end 97.04 66.29) (width 1) (layer B.Cu) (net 1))
 (segment (start 96.96 66.21) (end 74.79 66.21) (width 1) (layer B.Cu) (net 1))
 (segment (start 104.54 66.46) (end 104.79 66.21) (width 1) (layer B.Cu) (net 1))
 (segment (start 104.54 68.25) (end 104.54 66.46) (width 1) (layer B.Cu) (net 1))
 (segment (start 104.79 66.21) (end 96.96 66.21) (width 1) (layer B.Cu) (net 1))
 (segment (start 119.21 66.21) (end 104.79 66.21) (width 1) (layer B.Cu) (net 1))
 (segment (start 119.54 68.25) (end 119.54 66.96) (width 1) (layer B.Cu) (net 1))
 (segment (start 119.54 66.54) (end 119.54 66.96) (width 0.25) (layer B.Cu) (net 1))
 (segment (start 119.54 66.54) (end 119.21 66.21) (width 1) (layer B.Cu) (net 1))
 (segment (start 119.54 68.25) (end 119.54 66.54) (width 1) (layer B.Cu) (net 1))
 (segment (start 112.04 68.25) (end 112.04 66.54) (width 1) (layer B.Cu) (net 1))
 (segment (start 112.04 66.54) (end 112.04 66.21) (width 0.25) (layer B.Cu) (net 1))
 (segment (start 126.5 60.12) (end 126.5 67.25) (width 1) (layer B.Cu) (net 1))
 (segment (start 125.5 68.25) (end 119.54 68.25) (width 1) (layer B.Cu) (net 1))
 (segment (start 126.5 67.25) (end 125.5 68.25) (width 1) (layer B.Cu) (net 1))
 (segment (start 72 45.75) (end 72 46) (width 1) (layer B.Cu) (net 2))
 (segment (start 84.13 77.75) (end 84.13 76.13) (width 1) (layer B.Cu) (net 2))
 (segment (start 84.13 76.13) (end 82.5 74.5) (width 1) (layer B.Cu) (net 2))
 (segment (start 82.5 74.5) (end 74 74.5) (width 1) (layer B.Cu) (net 2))
 (segment (start 72 72.5) (end 72 69.25) (width 1) (layer B.Cu) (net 2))
 (segment (start 72 69.25) (end 72 68.25) (width 1) (layer B.Cu) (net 2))
 (segment (start 74 74.5) (end 72 72.5) (width 1) (layer B.Cu) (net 2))
 (segment (start 72 70.5) (end 72 69.25) (width 1) (layer B.Cu) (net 2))
 (segment (start 86.67 77.75) (end 86.67 75.42) (width 1) (layer B.Cu) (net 10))
 (segment (start 86.67 75.42) (end 82.75 71.5) (width 1) (layer B.Cu) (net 10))
 (segment (start 82.75 71.5) (end 81.25 71.5) (width 1) (layer B.Cu) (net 10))
 (segment (start 79.5 69.75) (end 79.5 68.25) (width 1) (layer B.Cu) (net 10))
 (segment (start 81.25 71.5) (end 79.5 69.75) (width 1) (layer B.Cu) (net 10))
 (segment (start 89.21 77.75) (end 89.21 73.96) (width 1) (layer B.Cu) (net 11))
 (segment (start 87 71.75) (end 87 68.25) (width 1) (layer B.Cu) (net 11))
 (segment (start 89.21 73.96) (end 87 71.75) (width 1) (layer B.Cu) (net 11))
 (segment (start 91.75 77.75) (end 91.75 74) (width 1) (layer B.Cu) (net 12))
 (segment (start 94.5 71.25) (end 94.5 68.25) (width 1) (layer B.Cu) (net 12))
 (segment (start 91.75 74) (end 94.5 71.25) (width 1) (layer B.Cu) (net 12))
 (segment (start 94.29 77.75) (end 94.29 75.96) (width 1) (layer B.Cu) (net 5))
 (segment (start 94.29 75.96) (end 98 72.25) (width 1) (layer B.Cu) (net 5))
 (segment (start 98 72.25) (end 100.75 72.25) (width 1) (layer B.Cu) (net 5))
 (segment (start 102 71) (end 102 68.25) (width 1) (layer B.Cu) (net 5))
 (segment (start 100.75 72.25) (end 102 71) (width 1) (layer B.Cu) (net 5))
 (segment (start 96.83 76.547919) (end 98.877919 74.5) (width 1) (layer B.Cu) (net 3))
 (segment (start 96.83 77.75) (end 96.83 76.547919) (width 1) (layer B.Cu) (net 3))
 (segment (start 98.877919 74.5) (end 106.75 74.5) (width 1) (layer B.Cu) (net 3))
 (segment (start 109.5 71.75) (end 109.5 68.25) (width 1) (layer B.Cu) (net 3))
 (segment (start 106.75 74.5) (end 109.5 71.75) (width 1) (layer B.Cu) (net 3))
 (segment (start 99.37 77.75) (end 112.25 77.75) (width 1) (layer B.Cu) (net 4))
 (segment (start 117 73) (end 117 68.25) (width 1) (layer B.Cu) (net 4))
 (segment (start 112.25 77.75) (end 117 73) (width 1) (layer B.Cu) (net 4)))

